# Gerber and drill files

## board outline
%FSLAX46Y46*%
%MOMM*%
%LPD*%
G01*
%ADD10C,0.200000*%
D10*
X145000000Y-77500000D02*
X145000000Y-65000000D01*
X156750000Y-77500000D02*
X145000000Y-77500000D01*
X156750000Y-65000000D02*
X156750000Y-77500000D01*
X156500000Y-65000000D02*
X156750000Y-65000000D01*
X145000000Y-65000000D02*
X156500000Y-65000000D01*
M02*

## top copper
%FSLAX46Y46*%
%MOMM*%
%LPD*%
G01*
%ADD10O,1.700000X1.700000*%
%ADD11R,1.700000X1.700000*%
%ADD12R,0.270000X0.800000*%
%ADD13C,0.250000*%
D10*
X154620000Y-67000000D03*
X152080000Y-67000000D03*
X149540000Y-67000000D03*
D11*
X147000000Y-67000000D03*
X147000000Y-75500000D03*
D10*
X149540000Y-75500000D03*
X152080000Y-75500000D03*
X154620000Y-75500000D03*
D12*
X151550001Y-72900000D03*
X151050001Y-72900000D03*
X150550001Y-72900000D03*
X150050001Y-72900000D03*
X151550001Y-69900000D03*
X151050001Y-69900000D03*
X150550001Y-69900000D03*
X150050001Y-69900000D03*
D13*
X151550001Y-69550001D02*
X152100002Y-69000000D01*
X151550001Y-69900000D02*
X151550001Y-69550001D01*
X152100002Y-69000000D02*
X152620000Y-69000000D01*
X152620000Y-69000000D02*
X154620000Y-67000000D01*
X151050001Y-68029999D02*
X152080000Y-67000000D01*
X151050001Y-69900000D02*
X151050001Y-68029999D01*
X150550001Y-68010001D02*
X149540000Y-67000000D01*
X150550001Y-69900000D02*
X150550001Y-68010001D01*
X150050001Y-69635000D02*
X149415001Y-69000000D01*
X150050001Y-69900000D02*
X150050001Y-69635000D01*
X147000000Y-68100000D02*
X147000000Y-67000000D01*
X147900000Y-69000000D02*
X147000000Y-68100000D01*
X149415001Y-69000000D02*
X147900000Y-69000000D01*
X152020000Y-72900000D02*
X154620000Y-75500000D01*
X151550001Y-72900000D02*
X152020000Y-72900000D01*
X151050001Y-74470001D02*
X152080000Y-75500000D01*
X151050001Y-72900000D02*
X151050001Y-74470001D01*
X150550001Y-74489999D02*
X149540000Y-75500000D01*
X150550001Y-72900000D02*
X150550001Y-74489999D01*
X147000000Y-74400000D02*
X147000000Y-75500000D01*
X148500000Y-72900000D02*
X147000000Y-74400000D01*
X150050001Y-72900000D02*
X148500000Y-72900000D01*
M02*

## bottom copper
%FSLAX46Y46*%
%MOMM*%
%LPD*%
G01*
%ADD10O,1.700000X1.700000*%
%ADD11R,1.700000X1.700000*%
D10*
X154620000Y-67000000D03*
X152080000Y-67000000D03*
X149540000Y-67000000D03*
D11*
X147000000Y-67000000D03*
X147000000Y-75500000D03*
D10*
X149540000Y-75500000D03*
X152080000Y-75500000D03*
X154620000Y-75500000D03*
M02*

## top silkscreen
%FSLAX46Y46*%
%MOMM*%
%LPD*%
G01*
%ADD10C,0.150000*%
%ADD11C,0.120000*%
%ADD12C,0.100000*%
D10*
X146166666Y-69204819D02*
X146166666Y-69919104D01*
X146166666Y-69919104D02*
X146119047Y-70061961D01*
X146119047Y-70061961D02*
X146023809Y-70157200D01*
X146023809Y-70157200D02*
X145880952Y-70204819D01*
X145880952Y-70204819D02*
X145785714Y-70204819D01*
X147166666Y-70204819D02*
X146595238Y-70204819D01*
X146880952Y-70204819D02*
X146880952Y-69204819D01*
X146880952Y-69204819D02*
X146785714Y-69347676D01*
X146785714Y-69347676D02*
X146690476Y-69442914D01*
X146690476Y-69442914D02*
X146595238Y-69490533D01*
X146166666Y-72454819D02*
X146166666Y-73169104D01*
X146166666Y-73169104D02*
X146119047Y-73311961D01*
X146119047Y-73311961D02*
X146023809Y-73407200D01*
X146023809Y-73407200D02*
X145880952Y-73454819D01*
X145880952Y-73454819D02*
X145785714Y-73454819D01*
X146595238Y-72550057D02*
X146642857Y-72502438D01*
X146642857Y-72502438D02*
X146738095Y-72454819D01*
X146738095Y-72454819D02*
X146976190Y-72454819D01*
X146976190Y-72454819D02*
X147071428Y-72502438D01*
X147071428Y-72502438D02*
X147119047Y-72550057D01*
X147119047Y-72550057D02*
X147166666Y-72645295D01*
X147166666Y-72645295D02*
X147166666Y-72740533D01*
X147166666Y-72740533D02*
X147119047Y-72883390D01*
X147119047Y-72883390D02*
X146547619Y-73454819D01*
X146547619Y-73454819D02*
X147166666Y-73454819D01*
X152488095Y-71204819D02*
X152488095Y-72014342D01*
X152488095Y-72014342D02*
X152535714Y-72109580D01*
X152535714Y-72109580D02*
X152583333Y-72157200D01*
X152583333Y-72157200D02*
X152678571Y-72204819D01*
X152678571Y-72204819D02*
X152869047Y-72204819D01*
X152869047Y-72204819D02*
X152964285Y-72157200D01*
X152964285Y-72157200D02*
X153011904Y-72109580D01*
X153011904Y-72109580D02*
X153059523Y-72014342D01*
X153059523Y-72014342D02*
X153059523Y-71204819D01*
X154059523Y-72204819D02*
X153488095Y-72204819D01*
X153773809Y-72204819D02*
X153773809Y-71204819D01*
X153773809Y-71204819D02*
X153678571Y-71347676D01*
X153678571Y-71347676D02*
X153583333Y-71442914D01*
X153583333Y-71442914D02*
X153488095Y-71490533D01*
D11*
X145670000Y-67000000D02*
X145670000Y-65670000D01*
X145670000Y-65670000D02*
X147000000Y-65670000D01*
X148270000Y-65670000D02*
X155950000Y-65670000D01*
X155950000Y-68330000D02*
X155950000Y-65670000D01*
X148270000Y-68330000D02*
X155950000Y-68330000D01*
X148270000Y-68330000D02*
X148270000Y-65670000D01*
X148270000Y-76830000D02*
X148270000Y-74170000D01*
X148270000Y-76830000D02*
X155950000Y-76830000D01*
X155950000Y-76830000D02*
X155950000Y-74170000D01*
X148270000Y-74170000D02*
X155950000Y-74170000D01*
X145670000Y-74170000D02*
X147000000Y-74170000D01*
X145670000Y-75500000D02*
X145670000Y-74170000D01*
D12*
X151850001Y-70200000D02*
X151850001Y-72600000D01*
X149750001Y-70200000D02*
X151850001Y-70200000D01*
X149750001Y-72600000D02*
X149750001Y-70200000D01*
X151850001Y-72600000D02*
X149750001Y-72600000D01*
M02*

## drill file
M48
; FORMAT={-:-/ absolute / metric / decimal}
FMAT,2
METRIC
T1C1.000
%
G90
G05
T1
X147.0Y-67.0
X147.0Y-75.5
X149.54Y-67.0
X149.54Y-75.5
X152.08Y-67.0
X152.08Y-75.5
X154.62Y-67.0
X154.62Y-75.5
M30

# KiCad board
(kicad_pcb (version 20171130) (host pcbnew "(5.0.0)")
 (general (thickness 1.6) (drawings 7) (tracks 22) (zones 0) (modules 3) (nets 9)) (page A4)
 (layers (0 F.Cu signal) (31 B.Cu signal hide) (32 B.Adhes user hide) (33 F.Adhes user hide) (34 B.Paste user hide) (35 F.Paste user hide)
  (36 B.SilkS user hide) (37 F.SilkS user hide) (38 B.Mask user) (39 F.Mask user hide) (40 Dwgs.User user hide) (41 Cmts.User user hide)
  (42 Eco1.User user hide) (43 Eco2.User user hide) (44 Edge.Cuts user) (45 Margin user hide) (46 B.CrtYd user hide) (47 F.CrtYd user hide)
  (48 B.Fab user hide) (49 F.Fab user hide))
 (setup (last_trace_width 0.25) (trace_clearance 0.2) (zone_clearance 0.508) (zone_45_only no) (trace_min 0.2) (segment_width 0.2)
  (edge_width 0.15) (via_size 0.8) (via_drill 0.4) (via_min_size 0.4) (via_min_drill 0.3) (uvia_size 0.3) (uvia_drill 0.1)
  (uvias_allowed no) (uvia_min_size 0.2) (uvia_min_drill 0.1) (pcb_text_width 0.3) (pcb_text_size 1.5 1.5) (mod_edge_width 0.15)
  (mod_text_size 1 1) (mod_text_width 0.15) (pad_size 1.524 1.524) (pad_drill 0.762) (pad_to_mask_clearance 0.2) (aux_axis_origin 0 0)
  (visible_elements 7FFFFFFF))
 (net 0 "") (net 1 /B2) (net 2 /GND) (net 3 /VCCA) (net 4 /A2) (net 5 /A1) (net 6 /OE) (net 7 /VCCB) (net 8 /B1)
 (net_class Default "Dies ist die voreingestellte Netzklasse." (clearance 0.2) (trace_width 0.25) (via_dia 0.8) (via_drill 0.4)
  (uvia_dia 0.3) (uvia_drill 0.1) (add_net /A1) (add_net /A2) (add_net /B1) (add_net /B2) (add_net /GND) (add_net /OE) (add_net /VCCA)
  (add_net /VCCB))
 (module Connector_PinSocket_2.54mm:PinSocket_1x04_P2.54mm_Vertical (layer F.Cu) (at 147 67 90)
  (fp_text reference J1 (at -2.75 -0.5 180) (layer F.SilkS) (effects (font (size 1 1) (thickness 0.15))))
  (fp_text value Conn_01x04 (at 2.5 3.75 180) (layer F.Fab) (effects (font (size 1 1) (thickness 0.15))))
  (fp_line (start 0 -1.33) (end 1.33 -1.33) (layer F.SilkS) (width 0.12))
  (fp_line (start 1.33 -1.33) (end 1.33 0) (layer F.SilkS) (width 0.12))
  (fp_line (start 1.33 1.27) (end 1.33 8.95) (layer F.SilkS) (width 0.12))
  (fp_line (start -1.33 8.95) (end 1.33 8.95) (layer F.SilkS) (width 0.12))
  (fp_line (start -1.33 1.27) (end -1.33 8.95) (layer F.SilkS) (width 0.12))
  (fp_line (start -1.33 1.27) (end 1.33 1.27) (layer F.SilkS) (width 0.12))
  (pad 4 thru_hole oval (at 0 7.62 90) (size 1.7 1.7) (drill 1) (layers *.Cu *.Mask) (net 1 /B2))
  (pad 3 thru_hole oval (at 0 5.08 90) (size 1.7 1.7) (drill 1) (layers *.Cu *.Mask) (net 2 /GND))
  (pad 2 thru_hole oval (at 0 2.54 90) (size 1.7 1.7) (drill 1) (layers *.Cu *.Mask) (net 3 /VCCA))
  (pad 1 thru_hole rect (at 0 0 90) (size 1.7 1.7) (drill 1) (layers *.Cu *.Mask) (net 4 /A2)))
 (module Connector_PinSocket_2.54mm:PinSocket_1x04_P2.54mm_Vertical (layer F.Cu) (at 147 75.5 90)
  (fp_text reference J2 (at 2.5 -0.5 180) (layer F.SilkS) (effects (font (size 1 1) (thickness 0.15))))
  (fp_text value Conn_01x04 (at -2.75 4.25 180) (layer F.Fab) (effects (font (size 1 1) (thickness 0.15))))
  (fp_line (start -1.33 1.27) (end 1.33 1.27) (layer F.SilkS) (width 0.12))
  (fp_line (start -1.33 1.27) (end -1.33 8.95) (layer F.SilkS) (width 0.12))
  (fp_line (start -1.33 8.95) (end 1.33 8.95) (layer F.SilkS) (width 0.12))
  (fp_line (start 1.33 1.27) (end 1.33 8.95) (layer F.SilkS) (width 0.12))
  (fp_line (start 1.33 -1.33) (end 1.33 0) (layer F.SilkS) (width 0.12))
  (fp_line (start 0 -1.33) (end 1.33 -1.33) (layer F.SilkS) (width 0.12))
  (pad 1 thru_hole rect (at 0 0 90) (size 1.7 1.7) (drill 1) (layers *.Cu *.Mask) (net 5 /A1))
  (pad 2 thru_hole oval (at 0 2.54 90) (size 1.7 1.7) (drill 1) (layers *.Cu *.Mask) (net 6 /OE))
  (pad 3 thru_hole oval (at 0 5.08 90) (size 1.7 1.7) (drill 1) (layers *.Cu *.Mask) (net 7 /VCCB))
  (pad 4 thru_hole oval (at 0 7.62 90) (size 1.7 1.7) (drill 1) (layers *.Cu *.Mask) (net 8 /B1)))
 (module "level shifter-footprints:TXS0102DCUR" (layer F.Cu) (at 150.800001 71.4 180)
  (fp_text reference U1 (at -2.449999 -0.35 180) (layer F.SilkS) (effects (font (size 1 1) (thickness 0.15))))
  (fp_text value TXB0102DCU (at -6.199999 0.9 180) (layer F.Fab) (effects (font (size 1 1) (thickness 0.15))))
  (fp_line (start -1.05 1.2) (end -1.05 -1.2) (layer F.SilkS) (width 0.1))
  (fp_line (start 1.05 1.2) (end -1.05 1.2) (layer F.SilkS) (width 0.1))
  (fp_line (start 1.05 -1.2) (end 1.05 1.2) (layer F.SilkS) (width 0.1))
  (fp_line (start -1.05 -1.2) (end 1.05 -1.2) (layer F.SilkS) (width 0.1))
  (pad 8 smd rect (at -0.75 -1.5 180) (size 0.27 0.8) (layers F.Cu F.Paste F.Mask) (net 8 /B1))
  (pad 7 smd rect (at -0.25 -1.5 180) (size 0.27 0.8) (layers F.Cu F.Paste F.Mask) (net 7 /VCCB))
  (pad 6 smd rect (at 0.25 -1.5 180) (size 0.27 0.8) (layers F.Cu F.Paste F.Mask) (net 6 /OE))
  (pad 5 smd rect (at 0.75 -1.5 180) (size 0.27 0.8) (layers F.Cu F.Paste F.Mask) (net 5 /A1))
  (pad 1 smd rect (at -0.75 1.5 180) (size 0.27 0.8) (layers F.Cu F.Paste F.Mask) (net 1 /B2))
  (pad 2 smd rect (at -0.25 1.5 180) (size 0.27 0.8) (layers F.Cu F.Paste F.Mask) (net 2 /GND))
  (pad 3 smd rect (at 0.25 1.5 180) (size 0.27 0.8) (layers F.Cu F.Paste F.Mask) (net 3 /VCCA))
  (pad 4 smd rect (at 0.75 1.5 180) (size 0.27 0.8) (layers F.Cu F.Paste F.Mask) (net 4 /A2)))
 (gr_line (start 145 77.5) (end 145 65) (layer Edge.Cuts) (width 0.2))
 (gr_line (start 156.75 77.5) (end 145 77.5) (layer Edge.Cuts) (width 0.2))
 (gr_line (start 156.75 65) (end 156.75 77.5) (layer Edge.Cuts) (width 0.2))
 (gr_line (start 156.5 65) (end 156.75 65) (layer Edge.Cuts) (width 0.2))
 (gr_line (start 145 65) (end 156.5 65) (layer Edge.Cuts) (width 0.2))
 (segment (start 151.550001 69.550001) (end 152.100002 69) (width 0.25) (layer F.Cu) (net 1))
 (segment (start 151.550001 69.9) (end 151.550001 69.550001) (width 0.25) (layer F.Cu) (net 1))
 (segment (start 152.100002 69) (end 152.62 69) (width 0.25) (layer F.Cu) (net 1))
 (segment (start 152.62 69) (end 154.62 67) (width 0.25) (layer F.Cu) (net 1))
 (segment (start 151.050001 68.029999) (end 152.08 67) (width 0.25) (layer F.Cu) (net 2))
 (segment (start 151.050001 69.9) (end 151.050001 68.029999) (width 0.25) (layer F.Cu) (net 2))
 (segment (start 150.550001 68.010001) (end 149.54 67) (width 0.25) (layer F.Cu) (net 3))
 (segment (start 150.550001 69.9) (end 150.550001 68.010001) (width 0.25) (layer F.Cu) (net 3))
 (segment (start 150.050001 69.635) (end 149.415001 69) (width 0.25) (layer F.Cu) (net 4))
 (segment (start 150.050001 69.9) (end 150.050001 69.635) (width 0.25) (layer F.Cu) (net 4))
 (segment (start 147 68.1) (end 147 67) (width 0.25) (layer F.Cu) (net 4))
 (segment (start 147.9 69) (end 147 68.1) (width 0.25) (layer F.Cu) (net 4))
 (segment (start 149.415001 69) (end 147.9 69) (width 0.25) (layer F.Cu) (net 4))
 (segment (start 152.02 72.9) (end 154.62 75.5) (width 0.25) (layer F.Cu) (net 8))
 (segment (start 151.550001 72.9) (end 152.02 72.9) (width 0.25) (layer F.Cu) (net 8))
 (segment (start 151.050001 74.470001) (end 152.08 75.5) (width 0.25) (layer F.Cu) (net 7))
 (segment (start 151.050001 72.9) (end 151.050001 74.470001) (width 0.25) (layer F.Cu) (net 7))
 (segment (start 150.550001 74.489999) (end 149.54 75.5) (width 0.25) (layer F.Cu) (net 6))
 (segment (start 150.550001 72.9) (end 150.550001 74.489999) (width 0.25) (layer F.Cu) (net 6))
 (segment (start 147 74.4) (end 147 75.5) (width 0.25) (layer F.Cu) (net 5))
 (segment (start 148.5 72.9) (end 147 74.4) (width 0.25) (layer F.Cu) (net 5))
 (segment (start 150.050001 72.9) (end 148.5 72.9) (width 0.25) (layer F.Cu) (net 5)))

